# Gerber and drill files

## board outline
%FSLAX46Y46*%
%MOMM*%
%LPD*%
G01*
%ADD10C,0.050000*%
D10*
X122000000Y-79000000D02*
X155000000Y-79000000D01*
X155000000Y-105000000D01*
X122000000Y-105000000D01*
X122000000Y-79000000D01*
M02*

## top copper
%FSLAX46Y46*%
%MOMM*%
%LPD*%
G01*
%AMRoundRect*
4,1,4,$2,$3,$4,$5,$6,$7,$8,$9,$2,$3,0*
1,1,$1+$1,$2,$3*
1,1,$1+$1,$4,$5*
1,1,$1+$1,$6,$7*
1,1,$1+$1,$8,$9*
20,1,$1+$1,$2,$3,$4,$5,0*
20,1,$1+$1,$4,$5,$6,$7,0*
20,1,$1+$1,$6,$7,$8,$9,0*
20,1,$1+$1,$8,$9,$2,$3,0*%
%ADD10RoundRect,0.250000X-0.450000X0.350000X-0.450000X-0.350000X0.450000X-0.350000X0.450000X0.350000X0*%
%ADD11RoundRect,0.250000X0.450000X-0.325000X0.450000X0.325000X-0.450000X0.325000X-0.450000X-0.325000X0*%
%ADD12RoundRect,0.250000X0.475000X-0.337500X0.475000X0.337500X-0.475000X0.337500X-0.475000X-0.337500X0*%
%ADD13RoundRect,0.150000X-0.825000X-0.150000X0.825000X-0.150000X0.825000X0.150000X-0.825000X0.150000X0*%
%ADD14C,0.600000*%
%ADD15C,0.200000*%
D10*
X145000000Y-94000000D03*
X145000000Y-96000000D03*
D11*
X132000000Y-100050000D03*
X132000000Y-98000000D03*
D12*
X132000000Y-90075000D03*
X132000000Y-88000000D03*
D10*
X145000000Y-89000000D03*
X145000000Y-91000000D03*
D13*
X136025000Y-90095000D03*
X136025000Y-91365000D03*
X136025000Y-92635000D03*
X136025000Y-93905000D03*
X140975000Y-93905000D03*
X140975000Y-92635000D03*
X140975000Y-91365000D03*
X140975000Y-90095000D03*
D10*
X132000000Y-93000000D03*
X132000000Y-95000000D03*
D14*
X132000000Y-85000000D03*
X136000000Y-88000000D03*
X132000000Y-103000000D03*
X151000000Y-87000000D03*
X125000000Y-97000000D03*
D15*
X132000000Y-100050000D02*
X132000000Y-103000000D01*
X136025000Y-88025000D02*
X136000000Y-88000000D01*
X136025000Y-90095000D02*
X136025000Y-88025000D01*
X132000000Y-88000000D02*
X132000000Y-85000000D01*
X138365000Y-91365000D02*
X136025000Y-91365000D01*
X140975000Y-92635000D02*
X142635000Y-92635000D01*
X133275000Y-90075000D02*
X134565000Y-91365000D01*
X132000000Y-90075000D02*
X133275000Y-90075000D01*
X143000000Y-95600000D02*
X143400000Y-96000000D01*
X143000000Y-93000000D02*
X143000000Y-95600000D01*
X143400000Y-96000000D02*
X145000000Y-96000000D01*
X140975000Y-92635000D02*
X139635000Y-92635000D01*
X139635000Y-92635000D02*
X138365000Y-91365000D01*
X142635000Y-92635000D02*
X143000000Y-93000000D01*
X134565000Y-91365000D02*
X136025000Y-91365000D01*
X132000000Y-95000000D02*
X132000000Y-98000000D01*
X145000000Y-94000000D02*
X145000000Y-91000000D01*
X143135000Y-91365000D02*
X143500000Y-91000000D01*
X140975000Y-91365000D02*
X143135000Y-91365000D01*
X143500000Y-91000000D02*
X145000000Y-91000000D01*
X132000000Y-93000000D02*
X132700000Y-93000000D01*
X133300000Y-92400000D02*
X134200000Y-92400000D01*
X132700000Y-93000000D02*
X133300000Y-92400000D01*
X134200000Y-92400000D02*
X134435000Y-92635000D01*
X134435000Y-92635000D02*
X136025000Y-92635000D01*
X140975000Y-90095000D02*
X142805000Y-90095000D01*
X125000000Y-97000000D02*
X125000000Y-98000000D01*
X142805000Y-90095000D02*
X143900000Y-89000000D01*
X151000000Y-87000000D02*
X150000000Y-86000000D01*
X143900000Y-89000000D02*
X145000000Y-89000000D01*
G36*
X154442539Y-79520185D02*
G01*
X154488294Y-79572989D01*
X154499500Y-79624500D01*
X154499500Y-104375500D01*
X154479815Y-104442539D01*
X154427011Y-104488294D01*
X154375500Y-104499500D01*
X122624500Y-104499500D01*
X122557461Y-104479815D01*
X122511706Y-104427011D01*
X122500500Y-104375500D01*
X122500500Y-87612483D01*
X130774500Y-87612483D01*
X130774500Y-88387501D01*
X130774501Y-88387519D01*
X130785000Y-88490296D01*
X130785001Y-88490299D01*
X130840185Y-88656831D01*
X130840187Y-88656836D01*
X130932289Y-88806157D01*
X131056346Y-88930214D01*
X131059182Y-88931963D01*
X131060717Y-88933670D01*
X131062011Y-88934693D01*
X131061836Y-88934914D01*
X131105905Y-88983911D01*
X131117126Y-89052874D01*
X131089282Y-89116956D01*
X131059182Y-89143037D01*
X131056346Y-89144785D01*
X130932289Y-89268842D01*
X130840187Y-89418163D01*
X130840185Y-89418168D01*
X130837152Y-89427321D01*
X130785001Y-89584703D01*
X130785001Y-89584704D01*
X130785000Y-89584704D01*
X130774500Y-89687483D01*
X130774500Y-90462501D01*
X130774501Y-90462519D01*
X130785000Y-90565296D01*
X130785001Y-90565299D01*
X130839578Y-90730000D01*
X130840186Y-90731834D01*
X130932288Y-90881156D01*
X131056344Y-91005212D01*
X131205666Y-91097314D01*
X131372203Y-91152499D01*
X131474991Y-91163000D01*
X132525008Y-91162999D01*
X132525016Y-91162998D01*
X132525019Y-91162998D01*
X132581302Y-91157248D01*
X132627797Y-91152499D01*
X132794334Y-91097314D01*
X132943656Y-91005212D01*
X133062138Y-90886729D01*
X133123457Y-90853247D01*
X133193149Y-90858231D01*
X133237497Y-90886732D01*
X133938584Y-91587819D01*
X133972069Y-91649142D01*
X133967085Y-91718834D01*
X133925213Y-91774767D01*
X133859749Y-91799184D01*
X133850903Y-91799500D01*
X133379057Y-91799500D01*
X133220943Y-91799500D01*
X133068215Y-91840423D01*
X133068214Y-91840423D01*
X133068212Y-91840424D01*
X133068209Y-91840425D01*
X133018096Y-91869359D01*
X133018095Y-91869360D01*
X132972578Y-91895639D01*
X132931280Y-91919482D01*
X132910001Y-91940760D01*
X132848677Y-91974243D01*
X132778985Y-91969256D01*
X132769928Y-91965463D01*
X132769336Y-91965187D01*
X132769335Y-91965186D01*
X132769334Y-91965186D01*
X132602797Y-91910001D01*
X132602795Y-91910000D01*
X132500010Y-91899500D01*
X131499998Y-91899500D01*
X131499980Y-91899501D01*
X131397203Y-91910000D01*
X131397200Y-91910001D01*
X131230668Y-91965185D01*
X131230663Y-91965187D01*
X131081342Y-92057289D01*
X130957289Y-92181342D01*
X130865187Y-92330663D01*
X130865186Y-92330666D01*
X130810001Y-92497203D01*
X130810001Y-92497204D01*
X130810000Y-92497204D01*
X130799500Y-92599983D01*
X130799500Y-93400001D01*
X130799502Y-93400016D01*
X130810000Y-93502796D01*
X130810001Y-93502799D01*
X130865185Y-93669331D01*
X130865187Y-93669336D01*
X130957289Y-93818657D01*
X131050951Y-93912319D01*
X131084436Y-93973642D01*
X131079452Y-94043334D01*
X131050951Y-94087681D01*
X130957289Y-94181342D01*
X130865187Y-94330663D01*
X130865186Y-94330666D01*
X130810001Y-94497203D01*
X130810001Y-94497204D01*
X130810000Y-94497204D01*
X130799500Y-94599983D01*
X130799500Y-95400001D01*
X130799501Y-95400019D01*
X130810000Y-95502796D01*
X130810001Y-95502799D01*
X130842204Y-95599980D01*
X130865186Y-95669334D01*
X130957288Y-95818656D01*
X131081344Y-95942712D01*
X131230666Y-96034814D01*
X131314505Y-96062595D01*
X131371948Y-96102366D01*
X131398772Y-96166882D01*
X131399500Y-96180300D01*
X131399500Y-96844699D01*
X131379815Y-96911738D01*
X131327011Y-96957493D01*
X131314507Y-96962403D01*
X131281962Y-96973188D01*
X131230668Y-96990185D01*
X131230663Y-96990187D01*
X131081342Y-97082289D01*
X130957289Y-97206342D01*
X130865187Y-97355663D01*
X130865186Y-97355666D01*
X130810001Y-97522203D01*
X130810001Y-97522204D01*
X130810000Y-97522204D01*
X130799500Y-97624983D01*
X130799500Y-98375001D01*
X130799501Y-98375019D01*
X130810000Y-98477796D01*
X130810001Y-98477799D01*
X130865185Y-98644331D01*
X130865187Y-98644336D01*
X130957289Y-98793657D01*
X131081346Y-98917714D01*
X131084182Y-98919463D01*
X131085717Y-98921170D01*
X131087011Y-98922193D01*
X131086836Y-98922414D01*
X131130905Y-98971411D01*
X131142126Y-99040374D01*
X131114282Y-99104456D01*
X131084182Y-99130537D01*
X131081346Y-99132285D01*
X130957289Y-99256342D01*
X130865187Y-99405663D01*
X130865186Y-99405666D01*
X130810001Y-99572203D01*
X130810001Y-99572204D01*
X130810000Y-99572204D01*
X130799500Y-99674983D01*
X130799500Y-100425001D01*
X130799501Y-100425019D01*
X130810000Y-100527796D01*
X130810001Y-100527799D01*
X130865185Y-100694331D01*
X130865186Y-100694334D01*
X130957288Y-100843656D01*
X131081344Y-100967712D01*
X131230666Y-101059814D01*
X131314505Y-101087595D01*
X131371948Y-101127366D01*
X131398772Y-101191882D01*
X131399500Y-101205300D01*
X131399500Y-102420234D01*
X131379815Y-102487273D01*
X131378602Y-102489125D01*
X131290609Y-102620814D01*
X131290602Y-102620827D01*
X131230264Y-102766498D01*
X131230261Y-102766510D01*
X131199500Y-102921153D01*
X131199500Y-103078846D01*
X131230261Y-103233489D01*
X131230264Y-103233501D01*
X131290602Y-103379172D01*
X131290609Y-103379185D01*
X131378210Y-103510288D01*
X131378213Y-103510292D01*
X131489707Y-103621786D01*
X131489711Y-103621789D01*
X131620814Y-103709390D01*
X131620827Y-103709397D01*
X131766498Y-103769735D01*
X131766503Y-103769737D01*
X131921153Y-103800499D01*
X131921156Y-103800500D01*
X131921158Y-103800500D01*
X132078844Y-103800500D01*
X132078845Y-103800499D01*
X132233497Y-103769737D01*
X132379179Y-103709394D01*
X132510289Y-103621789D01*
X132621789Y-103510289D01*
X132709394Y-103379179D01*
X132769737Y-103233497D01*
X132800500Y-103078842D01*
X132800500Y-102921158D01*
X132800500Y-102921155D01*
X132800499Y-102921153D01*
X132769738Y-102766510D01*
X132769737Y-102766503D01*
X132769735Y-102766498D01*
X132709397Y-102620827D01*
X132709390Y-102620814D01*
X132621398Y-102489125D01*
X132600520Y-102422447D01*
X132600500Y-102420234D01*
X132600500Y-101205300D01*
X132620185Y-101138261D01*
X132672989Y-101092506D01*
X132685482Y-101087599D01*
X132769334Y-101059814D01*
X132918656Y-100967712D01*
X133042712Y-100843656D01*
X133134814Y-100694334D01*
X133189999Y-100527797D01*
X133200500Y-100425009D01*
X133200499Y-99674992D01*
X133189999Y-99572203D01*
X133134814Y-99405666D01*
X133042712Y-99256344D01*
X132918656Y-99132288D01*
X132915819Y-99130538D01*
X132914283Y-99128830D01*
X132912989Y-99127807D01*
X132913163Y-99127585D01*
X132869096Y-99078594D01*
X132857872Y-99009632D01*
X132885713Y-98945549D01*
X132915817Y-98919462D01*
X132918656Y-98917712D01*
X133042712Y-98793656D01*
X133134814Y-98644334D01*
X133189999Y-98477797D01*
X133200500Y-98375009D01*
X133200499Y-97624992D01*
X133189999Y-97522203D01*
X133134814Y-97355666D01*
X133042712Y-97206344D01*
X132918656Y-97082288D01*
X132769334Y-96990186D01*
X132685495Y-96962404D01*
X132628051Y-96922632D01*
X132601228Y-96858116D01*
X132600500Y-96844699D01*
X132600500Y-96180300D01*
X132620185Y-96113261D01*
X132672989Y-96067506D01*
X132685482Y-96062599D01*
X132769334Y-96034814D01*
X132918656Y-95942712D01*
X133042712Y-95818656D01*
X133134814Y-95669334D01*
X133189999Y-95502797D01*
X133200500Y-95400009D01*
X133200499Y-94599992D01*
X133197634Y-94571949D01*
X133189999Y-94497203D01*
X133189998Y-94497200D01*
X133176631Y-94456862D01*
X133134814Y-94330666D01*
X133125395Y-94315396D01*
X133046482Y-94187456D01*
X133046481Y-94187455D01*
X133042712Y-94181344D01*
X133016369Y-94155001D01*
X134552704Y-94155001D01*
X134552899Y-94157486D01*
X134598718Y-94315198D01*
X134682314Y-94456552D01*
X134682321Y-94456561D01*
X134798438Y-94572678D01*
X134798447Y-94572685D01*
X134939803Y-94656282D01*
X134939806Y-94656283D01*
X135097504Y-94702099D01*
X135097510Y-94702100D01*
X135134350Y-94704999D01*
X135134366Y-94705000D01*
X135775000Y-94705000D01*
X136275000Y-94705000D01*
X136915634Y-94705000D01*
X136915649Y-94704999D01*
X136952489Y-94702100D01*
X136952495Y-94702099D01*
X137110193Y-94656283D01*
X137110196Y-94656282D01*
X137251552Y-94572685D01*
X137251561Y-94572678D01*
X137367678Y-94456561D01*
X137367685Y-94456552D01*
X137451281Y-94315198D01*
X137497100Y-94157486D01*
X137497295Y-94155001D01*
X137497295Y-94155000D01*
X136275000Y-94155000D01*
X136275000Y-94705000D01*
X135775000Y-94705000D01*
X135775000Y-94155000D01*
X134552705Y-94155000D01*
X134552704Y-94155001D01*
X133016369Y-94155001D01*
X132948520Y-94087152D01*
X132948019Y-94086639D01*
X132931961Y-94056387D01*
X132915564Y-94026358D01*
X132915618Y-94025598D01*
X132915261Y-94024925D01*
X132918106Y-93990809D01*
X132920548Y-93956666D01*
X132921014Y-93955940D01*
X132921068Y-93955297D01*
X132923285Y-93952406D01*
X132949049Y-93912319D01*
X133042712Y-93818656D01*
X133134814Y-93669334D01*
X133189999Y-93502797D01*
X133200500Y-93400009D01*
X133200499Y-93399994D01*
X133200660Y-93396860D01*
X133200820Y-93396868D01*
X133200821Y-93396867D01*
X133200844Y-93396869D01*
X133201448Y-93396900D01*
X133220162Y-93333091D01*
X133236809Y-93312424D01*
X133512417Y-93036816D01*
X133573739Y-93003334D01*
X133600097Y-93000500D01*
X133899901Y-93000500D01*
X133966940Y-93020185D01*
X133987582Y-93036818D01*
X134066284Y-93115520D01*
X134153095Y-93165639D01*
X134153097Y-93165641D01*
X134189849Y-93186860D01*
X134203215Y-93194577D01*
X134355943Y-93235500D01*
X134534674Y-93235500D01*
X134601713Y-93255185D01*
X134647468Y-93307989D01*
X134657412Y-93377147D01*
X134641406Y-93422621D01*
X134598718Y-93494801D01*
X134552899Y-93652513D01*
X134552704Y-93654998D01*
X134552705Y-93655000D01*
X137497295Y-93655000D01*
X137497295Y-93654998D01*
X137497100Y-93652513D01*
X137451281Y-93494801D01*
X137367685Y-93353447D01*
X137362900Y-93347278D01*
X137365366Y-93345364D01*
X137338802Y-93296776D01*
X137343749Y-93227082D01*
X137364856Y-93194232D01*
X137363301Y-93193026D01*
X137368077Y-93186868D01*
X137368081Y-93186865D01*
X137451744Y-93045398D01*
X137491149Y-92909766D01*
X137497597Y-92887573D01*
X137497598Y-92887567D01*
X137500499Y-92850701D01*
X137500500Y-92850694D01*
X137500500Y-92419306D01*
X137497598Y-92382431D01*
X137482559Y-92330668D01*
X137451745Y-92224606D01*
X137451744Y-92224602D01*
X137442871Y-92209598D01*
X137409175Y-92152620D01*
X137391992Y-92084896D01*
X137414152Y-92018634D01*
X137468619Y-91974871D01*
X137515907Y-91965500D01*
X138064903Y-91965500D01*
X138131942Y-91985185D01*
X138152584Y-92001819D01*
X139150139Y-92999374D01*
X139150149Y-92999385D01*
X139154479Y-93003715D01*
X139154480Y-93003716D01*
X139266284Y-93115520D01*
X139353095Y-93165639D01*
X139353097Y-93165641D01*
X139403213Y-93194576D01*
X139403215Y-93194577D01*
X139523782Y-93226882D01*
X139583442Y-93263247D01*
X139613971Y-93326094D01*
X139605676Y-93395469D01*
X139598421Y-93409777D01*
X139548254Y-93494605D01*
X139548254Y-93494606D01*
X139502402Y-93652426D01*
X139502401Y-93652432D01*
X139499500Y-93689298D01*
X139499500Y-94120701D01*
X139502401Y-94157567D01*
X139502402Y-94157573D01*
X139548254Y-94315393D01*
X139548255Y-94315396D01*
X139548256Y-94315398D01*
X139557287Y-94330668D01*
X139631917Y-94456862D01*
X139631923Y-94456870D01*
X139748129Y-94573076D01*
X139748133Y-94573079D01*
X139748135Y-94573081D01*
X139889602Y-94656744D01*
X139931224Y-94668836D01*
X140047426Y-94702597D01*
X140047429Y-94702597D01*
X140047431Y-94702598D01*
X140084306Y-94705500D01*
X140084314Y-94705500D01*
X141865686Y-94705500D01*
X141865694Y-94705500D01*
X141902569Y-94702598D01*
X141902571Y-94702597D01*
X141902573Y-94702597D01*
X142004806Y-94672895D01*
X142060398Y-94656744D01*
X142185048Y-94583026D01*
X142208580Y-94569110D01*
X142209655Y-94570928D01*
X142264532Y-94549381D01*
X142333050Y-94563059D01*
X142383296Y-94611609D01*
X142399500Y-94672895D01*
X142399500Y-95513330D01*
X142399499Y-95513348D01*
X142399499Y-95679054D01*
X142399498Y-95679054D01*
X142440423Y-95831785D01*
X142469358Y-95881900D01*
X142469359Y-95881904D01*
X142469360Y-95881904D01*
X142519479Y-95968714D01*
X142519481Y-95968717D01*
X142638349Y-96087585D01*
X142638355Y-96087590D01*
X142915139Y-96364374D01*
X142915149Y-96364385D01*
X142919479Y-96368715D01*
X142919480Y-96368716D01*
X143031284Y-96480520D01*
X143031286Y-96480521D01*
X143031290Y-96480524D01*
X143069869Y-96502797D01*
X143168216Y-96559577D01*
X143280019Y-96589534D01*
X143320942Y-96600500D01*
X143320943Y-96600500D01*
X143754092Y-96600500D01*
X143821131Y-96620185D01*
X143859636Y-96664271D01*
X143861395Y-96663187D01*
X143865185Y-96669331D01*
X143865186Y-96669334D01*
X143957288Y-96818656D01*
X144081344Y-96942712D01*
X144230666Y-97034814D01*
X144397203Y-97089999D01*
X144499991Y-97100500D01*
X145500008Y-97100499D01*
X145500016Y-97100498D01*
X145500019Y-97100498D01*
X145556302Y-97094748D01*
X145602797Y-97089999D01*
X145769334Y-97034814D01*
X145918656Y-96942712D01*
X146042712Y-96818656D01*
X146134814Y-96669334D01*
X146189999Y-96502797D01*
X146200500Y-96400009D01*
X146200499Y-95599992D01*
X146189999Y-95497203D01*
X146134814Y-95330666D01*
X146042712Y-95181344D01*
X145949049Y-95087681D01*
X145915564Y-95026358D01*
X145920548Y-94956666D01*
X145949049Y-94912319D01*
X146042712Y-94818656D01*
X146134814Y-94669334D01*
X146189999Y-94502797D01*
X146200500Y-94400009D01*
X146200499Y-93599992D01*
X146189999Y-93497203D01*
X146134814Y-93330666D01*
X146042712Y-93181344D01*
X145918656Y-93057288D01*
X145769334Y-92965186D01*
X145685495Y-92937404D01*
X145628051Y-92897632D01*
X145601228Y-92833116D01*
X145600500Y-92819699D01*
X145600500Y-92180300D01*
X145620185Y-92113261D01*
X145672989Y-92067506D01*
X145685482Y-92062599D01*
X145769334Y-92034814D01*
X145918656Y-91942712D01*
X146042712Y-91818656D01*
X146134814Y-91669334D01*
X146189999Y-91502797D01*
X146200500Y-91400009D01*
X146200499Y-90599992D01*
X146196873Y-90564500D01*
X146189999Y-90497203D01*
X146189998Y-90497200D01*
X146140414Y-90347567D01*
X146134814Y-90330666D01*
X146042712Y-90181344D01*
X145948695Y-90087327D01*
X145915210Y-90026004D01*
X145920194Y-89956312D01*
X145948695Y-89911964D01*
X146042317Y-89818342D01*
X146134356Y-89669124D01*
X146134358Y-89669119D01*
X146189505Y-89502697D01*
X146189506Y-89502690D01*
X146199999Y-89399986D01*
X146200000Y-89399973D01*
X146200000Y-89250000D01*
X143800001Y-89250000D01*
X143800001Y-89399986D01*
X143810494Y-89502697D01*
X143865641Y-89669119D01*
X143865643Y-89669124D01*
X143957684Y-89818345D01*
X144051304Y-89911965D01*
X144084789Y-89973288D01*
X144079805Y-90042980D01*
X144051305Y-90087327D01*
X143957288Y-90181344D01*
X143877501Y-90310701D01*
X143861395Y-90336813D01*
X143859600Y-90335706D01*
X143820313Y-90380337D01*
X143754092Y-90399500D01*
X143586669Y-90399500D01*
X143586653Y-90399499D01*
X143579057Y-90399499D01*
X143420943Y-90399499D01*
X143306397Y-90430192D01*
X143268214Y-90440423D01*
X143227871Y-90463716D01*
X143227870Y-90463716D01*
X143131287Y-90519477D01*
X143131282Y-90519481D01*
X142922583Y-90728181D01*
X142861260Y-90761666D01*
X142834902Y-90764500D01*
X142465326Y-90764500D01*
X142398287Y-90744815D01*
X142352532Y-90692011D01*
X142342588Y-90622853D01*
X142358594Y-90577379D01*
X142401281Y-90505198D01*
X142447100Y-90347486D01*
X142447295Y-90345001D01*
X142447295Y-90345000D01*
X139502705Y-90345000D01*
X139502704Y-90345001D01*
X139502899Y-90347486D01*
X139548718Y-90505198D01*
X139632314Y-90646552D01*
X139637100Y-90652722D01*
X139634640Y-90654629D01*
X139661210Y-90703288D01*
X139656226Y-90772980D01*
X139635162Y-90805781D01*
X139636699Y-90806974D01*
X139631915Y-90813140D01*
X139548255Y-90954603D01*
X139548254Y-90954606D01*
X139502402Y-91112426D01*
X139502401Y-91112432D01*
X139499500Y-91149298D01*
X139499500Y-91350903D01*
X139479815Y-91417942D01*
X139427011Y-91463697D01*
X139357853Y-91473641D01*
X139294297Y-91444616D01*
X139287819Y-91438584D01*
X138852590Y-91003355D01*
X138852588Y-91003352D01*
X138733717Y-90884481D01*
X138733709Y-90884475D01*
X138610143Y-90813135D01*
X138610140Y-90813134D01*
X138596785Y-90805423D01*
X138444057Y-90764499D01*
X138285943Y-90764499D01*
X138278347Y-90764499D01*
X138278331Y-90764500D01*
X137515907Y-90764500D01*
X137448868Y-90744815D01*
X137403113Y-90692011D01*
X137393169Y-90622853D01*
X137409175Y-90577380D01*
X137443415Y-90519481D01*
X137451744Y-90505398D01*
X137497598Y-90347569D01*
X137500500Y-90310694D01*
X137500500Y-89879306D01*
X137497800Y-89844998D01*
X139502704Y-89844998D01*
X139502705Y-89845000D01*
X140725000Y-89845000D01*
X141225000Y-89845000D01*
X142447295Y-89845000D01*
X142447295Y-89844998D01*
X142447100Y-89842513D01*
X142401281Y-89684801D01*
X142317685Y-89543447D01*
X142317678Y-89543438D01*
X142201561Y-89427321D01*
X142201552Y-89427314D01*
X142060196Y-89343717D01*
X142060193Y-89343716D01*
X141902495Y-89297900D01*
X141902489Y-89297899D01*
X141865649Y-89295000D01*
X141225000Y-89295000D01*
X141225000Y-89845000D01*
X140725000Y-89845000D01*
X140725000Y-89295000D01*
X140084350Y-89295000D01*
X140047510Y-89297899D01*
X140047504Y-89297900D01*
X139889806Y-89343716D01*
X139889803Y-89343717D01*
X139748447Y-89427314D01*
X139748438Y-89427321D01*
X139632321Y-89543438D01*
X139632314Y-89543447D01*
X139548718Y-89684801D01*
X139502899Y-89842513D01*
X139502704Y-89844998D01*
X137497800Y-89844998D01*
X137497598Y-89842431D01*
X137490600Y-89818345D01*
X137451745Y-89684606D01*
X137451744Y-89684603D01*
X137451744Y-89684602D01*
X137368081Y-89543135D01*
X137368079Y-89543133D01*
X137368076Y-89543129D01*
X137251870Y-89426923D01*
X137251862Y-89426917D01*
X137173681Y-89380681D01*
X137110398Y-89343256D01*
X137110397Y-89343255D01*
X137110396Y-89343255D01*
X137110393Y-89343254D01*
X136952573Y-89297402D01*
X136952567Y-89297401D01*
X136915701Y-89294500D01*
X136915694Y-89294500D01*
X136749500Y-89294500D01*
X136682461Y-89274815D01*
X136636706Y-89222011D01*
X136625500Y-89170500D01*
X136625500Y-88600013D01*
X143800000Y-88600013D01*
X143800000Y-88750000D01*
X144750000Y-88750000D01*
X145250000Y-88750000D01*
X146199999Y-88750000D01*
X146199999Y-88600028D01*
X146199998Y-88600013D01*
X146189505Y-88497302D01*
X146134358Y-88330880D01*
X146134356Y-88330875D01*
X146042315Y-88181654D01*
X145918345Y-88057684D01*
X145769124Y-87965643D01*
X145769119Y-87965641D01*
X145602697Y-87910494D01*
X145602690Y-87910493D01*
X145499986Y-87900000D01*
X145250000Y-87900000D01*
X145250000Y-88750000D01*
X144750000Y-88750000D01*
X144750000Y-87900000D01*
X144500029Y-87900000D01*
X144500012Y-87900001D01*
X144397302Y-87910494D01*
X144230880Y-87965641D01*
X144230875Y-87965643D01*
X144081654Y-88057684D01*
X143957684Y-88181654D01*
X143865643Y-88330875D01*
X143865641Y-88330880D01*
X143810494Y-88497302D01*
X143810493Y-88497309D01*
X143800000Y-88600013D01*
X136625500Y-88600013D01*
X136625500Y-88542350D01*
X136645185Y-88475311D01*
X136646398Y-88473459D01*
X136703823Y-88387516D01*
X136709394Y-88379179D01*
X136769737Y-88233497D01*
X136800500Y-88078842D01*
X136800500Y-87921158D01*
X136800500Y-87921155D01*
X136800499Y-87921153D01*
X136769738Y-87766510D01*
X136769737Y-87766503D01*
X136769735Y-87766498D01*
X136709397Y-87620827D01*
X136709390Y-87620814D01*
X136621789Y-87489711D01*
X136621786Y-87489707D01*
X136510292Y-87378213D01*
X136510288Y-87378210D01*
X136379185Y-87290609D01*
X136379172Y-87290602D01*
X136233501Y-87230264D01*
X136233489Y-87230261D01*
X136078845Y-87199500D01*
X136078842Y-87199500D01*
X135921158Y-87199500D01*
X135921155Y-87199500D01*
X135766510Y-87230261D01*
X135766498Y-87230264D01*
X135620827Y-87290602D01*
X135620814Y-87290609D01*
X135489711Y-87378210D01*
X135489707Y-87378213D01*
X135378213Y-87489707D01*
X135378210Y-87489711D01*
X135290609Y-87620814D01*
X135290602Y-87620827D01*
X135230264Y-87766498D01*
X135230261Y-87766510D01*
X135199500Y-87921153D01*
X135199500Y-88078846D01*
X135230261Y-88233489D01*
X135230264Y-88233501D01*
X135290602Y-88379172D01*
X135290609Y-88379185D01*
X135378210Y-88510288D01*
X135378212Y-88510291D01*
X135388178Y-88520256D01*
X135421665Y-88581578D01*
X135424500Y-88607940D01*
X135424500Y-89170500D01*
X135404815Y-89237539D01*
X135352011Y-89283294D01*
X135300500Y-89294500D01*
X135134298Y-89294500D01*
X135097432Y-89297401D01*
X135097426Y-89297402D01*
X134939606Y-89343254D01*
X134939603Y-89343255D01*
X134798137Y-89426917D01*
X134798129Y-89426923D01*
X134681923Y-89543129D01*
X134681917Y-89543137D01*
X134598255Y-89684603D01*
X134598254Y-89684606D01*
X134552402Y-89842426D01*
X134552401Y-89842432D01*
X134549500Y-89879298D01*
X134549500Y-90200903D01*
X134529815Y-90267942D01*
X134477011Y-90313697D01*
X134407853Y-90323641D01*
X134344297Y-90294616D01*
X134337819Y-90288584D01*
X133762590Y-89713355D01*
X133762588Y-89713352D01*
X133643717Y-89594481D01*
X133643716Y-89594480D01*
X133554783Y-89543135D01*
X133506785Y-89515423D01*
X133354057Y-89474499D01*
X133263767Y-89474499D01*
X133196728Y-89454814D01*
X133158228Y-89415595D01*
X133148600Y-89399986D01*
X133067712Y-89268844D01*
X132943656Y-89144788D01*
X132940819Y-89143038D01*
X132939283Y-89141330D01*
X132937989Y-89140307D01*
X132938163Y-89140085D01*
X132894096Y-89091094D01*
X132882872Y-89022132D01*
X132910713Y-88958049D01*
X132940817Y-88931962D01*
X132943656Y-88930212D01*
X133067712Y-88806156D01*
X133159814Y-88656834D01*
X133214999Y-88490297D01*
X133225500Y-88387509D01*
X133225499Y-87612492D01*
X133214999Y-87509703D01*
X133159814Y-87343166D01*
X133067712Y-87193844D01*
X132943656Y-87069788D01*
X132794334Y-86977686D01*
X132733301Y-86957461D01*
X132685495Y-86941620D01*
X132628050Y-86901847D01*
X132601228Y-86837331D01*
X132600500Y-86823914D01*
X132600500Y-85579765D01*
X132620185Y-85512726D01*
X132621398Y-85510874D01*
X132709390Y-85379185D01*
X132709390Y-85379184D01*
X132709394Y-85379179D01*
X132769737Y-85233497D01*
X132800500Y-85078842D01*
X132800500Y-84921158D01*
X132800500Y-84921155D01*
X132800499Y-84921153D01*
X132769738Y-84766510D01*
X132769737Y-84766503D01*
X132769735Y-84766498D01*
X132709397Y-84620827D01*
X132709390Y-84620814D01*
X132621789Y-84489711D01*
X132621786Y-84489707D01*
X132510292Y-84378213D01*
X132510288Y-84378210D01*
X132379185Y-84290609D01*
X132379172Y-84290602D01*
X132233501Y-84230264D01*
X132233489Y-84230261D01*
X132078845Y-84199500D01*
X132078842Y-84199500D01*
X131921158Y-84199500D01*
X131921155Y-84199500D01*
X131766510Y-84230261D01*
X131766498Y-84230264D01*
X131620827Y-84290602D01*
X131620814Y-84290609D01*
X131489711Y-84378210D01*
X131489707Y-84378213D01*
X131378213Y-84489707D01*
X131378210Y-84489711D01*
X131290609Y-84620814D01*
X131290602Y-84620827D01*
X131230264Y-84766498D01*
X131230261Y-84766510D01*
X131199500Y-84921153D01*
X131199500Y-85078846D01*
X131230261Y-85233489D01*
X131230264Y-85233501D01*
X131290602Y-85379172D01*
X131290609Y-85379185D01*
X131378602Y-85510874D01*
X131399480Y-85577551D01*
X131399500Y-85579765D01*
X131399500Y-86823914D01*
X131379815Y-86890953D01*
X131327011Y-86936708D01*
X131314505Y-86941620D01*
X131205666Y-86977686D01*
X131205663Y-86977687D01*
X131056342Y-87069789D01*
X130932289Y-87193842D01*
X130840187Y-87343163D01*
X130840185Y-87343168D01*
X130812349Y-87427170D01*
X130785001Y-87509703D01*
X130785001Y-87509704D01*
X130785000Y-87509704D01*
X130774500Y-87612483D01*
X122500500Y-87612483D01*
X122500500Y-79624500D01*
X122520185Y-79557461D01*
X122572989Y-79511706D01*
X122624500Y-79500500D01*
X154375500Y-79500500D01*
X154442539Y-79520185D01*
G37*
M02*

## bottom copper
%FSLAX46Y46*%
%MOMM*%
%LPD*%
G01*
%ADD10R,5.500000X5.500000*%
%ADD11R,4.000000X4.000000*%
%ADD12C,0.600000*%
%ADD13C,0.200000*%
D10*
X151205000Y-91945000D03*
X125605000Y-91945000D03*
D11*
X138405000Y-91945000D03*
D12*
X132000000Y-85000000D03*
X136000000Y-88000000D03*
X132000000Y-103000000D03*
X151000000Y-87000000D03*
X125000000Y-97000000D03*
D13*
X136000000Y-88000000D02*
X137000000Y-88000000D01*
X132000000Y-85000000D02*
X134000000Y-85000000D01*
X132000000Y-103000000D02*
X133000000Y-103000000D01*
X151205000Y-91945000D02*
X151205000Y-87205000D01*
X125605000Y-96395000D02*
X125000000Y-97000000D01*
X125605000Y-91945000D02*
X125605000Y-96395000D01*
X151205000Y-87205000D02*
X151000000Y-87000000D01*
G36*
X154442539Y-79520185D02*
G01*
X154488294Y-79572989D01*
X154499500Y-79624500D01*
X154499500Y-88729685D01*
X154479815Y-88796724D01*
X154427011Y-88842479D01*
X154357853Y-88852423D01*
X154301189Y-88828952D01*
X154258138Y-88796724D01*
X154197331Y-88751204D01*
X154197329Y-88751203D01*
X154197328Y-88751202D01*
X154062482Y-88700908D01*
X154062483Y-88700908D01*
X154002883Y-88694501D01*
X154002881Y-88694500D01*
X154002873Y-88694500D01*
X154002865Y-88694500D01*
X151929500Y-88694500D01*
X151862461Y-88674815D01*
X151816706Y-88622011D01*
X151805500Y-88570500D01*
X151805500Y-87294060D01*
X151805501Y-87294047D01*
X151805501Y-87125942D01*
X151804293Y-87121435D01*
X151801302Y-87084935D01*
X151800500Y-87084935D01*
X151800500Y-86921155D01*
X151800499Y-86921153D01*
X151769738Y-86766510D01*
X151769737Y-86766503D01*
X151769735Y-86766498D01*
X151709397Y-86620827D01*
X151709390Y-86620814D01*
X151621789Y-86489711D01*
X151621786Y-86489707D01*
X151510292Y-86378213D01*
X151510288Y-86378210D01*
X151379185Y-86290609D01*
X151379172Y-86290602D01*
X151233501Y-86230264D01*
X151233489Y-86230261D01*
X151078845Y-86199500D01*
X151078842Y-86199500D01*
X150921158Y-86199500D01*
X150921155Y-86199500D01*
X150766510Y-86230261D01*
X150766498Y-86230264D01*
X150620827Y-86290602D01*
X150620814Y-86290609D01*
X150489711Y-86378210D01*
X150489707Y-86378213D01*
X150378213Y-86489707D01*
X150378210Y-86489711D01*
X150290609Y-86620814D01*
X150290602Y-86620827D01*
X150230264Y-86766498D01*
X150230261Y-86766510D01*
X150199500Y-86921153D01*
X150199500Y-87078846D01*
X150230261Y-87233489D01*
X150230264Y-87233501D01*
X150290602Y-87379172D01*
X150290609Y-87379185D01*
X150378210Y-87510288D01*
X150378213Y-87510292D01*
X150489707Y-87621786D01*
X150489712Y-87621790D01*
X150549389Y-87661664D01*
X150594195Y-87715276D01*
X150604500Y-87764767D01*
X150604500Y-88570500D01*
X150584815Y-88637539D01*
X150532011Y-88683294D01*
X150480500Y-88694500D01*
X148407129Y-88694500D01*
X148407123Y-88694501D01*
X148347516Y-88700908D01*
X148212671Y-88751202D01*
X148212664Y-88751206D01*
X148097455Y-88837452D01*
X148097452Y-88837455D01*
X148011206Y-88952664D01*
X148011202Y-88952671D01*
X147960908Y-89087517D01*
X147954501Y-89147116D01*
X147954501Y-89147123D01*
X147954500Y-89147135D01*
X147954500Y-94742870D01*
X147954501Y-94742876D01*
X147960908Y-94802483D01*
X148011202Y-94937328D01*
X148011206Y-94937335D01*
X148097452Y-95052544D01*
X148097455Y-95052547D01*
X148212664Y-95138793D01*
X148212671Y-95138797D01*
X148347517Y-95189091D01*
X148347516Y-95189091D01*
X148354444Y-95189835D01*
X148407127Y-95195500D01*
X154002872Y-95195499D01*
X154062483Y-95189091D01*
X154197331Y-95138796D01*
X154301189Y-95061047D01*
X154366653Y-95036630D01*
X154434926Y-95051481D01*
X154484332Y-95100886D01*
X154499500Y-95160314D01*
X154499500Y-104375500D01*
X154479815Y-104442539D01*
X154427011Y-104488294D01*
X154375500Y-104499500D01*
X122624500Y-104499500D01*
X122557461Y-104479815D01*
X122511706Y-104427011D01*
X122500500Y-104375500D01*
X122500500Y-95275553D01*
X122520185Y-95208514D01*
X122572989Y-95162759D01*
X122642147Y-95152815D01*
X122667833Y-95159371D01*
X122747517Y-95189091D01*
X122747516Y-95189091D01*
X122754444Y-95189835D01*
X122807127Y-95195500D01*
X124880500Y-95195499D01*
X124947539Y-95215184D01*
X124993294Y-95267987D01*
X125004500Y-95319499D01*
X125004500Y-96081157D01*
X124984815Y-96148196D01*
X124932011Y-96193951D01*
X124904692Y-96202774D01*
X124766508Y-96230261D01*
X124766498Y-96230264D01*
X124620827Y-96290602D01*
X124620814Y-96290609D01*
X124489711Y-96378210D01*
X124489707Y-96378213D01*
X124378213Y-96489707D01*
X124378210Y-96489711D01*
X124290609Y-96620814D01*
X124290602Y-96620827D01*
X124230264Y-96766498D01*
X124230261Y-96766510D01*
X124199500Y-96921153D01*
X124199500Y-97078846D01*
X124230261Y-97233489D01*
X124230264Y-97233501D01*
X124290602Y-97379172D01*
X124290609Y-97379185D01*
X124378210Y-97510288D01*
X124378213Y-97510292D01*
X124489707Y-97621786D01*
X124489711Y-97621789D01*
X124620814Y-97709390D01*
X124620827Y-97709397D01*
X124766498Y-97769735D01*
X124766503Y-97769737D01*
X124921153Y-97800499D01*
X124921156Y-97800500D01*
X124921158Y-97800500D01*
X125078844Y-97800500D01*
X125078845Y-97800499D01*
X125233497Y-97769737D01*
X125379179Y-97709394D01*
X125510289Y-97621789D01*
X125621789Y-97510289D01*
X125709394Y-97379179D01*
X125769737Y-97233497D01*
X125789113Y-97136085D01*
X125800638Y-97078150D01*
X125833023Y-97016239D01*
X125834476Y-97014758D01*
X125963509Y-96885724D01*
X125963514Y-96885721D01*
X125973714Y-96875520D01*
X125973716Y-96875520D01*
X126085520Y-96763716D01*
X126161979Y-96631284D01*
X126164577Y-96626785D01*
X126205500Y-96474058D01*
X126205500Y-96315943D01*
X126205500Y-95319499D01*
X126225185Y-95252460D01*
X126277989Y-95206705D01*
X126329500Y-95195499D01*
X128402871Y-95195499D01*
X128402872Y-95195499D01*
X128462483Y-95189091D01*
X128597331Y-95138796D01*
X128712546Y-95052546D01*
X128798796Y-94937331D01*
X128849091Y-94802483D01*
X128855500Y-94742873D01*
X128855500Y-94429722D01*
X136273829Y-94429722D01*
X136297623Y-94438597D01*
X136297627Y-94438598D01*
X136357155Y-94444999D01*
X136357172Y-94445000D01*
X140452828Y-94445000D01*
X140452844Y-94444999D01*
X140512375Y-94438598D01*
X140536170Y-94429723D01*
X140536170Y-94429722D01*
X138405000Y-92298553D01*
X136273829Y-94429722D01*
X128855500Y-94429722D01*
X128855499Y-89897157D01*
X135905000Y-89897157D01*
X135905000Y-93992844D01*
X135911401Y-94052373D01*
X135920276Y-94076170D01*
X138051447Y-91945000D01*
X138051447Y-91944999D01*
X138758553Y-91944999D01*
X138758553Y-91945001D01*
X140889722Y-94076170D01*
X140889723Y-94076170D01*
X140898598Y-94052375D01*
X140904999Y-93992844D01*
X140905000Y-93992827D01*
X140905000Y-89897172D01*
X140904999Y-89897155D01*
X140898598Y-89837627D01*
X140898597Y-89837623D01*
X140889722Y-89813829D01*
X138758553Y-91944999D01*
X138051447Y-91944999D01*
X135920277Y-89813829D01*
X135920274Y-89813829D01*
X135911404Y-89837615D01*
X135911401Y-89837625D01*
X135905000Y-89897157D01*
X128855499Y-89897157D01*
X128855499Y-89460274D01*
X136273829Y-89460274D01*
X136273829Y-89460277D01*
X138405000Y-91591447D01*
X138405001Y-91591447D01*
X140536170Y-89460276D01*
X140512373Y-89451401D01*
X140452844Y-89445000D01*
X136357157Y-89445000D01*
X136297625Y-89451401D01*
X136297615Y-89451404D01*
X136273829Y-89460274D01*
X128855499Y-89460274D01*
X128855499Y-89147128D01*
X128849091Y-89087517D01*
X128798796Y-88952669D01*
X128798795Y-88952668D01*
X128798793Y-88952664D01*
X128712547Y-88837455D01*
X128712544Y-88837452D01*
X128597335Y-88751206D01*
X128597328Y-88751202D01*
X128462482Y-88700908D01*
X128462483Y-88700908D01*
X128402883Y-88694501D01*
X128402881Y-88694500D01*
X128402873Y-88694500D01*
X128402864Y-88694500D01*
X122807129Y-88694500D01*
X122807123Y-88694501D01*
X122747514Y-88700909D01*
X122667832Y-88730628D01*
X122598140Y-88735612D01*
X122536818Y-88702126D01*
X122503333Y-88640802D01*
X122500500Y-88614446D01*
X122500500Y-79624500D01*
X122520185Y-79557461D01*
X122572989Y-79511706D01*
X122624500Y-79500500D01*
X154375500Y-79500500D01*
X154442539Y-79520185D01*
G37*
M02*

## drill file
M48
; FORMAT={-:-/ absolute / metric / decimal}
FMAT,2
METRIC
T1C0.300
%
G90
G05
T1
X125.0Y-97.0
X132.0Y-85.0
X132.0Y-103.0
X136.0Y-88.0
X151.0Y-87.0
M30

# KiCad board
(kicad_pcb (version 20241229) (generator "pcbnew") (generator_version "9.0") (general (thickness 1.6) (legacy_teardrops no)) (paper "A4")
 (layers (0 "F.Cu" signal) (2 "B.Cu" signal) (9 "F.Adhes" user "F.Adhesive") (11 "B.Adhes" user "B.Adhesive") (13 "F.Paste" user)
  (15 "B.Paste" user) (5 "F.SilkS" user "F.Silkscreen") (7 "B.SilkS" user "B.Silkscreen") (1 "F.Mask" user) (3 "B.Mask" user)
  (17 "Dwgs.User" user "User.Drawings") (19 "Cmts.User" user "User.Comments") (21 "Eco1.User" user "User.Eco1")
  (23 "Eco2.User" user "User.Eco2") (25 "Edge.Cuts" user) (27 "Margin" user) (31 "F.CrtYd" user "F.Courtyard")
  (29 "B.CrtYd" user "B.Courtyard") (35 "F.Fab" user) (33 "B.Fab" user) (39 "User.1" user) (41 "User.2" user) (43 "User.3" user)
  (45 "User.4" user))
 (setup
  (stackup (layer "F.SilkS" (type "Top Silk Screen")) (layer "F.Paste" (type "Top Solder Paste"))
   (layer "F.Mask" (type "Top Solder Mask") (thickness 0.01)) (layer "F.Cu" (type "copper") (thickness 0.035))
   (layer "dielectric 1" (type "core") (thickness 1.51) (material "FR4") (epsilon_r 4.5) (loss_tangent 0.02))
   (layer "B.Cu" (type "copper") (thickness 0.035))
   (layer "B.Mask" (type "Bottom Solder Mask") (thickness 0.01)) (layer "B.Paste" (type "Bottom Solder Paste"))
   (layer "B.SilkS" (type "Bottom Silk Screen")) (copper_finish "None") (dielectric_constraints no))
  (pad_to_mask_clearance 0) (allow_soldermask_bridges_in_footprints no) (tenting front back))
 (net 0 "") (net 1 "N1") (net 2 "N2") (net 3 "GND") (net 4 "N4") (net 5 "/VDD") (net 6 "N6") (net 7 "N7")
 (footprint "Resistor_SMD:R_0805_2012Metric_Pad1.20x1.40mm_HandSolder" (layer "F.Cu") (at 145 95 -90)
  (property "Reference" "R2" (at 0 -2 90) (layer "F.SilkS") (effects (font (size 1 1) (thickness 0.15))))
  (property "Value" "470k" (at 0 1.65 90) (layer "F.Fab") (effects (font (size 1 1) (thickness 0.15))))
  (pad "1" smd roundrect (at -1 0 270) (size 1.2 1.4) (layers "F.Cu" "F.Mask" "F.Paste") (roundrect_rratio 0.208333) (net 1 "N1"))
  (pad "2" smd roundrect (at 1 0 270) (size 1.2 1.4) (layers "F.Cu" "F.Mask" "F.Paste") (roundrect_rratio 0.208333) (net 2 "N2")))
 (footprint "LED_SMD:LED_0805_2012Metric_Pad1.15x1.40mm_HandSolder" (layer "F.Cu") (at 132 99.025 90)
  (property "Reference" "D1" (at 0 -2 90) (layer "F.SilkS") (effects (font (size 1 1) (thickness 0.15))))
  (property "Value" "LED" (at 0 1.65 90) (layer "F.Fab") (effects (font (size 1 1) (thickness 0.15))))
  (pad "1" smd roundrect (at -1.025 0 90) (size 1.15 1.4) (layers "F.Cu" "F.Mask" "F.Paste") (roundrect_rratio 0.217391) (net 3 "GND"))
  (pad "2" smd roundrect (at 1.025 0 90) (size 1.15 1.4) (layers "F.Cu" "F.Mask" "F.Paste") (roundrect_rratio 0.217391) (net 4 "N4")))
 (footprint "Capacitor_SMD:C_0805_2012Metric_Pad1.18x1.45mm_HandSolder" (layer "F.Cu") (at 132 89.0375 90)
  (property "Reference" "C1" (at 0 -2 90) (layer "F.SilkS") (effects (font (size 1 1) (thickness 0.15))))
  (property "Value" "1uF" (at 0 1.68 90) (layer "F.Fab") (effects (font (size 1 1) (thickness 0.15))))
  (pad "1" smd roundrect (at -1.0375 0 90) (size 1.175 1.45) (layers "F.Cu" "F.Mask" "F.Paste") (roundrect_rratio 0.212766) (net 2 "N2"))
  (pad "2" smd roundrect (at 1.0375 0 90) (size 1.175 1.45) (layers "F.Cu" "F.Mask" "F.Paste") (roundrect_rratio 0.212766) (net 3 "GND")))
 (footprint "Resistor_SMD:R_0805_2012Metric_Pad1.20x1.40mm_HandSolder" (layer "F.Cu") (at 145 90 -90)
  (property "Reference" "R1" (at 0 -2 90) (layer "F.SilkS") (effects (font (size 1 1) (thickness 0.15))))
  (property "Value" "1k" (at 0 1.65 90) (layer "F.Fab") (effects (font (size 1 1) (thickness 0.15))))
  (pad "1" smd roundrect (at -1 0 270) (size 1.2 1.4) (layers "F.Cu" "F.Mask" "F.Paste") (roundrect_rratio 0.208333) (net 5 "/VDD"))
  (pad "2" smd roundrect (at 1 0 270) (size 1.2 1.4) (layers "F.Cu" "F.Mask" "F.Paste") (roundrect_rratio 0.208333) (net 1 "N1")))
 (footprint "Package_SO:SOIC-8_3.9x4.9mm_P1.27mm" (layer "F.Cu") (at 138.5 92)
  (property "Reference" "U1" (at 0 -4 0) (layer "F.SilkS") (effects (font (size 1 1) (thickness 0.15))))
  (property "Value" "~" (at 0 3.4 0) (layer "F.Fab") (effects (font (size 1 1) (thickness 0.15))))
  (pad "1" smd roundrect (at -2.475 -1.905) (size 1.95 0.6) (layers "F.Cu" "F.Mask" "F.Paste") (roundrect_rratio 0.25) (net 3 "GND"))
  (pad "2" smd roundrect (at -2.475 -0.635) (size 1.95 0.6) (layers "F.Cu" "F.Mask" "F.Paste") (roundrect_rratio 0.25) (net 2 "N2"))
  (pad "3" smd roundrect (at -2.475 0.635) (size 1.95 0.6) (layers "F.Cu" "F.Mask" "F.Paste") (roundrect_rratio 0.25) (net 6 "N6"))
  (pad "4" smd roundrect (at -2.475 1.905) (size 1.95 0.6) (layers "F.Cu" "F.Mask" "F.Paste") (roundrect_rratio 0.25) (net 5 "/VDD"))
  (pad "5" smd roundrect (at 2.475 1.905) (size 1.95 0.6) (layers "F.Cu" "F.Mask" "F.Paste") (roundrect_rratio 0.25) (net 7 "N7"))
  (pad "6" smd roundrect (at 2.475 0.635) (size 1.95 0.6) (layers "F.Cu" "F.Mask" "F.Paste") (roundrect_rratio 0.25) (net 2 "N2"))
  (pad "7" smd roundrect (at 2.475 -0.635) (size 1.95 0.6) (layers "F.Cu" "F.Mask" "F.Paste") (roundrect_rratio 0.25) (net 1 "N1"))
  (pad "8" smd roundrect (at 2.475 -1.905) (size 1.95 0.6) (layers "F.Cu" "F.Mask" "F.Paste") (roundrect_rratio 0.25) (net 5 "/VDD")))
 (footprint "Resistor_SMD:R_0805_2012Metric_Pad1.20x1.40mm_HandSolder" (layer "F.Cu") (at 132 94 -90)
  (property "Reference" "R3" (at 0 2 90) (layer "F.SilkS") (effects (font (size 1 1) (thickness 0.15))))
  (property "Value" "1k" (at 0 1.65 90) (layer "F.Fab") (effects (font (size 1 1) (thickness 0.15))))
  (pad "1" smd roundrect (at -1 0 270) (size 1.2 1.4) (layers "F.Cu" "F.Mask" "F.Paste") (roundrect_rratio 0.208333) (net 6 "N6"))
  (pad "2" smd roundrect (at 1 0 270) (size 1.2 1.4) (layers "F.Cu" "F.Mask" "F.Paste") (roundrect_rratio 0.208333) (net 4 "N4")))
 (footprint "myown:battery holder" (layer "B.Cu") (at 138.405 91.945 180)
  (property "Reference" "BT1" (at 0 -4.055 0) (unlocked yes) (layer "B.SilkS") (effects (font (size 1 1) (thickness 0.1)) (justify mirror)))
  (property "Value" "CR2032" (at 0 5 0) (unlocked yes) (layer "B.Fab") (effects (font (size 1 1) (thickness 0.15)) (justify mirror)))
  (pad "1" smd rect (at -12.8 0 180) (size 5.5 5.5) (layers "B.Cu" "B.Mask" "B.Paste") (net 5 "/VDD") (thermal_bridge_angle 45))
  (pad "1" smd rect (at 12.8 0 180) (size 5.5 5.5) (layers "B.Cu" "B.Mask" "B.Paste") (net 5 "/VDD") (thermal_bridge_angle 45))
  (pad "2" smd rect (at 0 0 180) (size 4 4) (layers "B.Cu" "B.Mask" "B.Paste") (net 3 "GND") (thermal_bridge_angle 45)))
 (gr_rect (start 122 79) (end 155 105) (stroke (width 0.05) (type default)) (fill no) (layer "Edge.Cuts"))
 (segment (start 132 100.05) (end 132 103) (width 0.2) (layer "F.Cu") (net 3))
 (segment (start 136.025 88.025) (end 136 88) (width 0.2) (layer "F.Cu") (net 3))
 (segment (start 136.025 90.095) (end 136.025 88.025) (width 0.2) (layer "F.Cu") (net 3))
 (segment (start 132 88) (end 132 85) (width 0.2) (layer "F.Cu") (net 3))
 (via (at 132 85) (size 0.6) (drill 0.3) (layers "F.Cu" "B.Cu") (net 3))
 (via (at 136 88) (size 0.6) (drill 0.3) (layers "F.Cu" "B.Cu") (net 3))
 (via (at 132 103) (size 0.6) (drill 0.3) (layers "F.Cu" "B.Cu") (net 3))
 (segment (start 136 88) (end 137 88) (width 0.2) (layer "B.Cu") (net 3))
 (segment (start 132 85) (end 134 85) (width 0.2) (layer "B.Cu") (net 3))
 (segment (start 132 103) (end 133 103) (width 0.2) (layer "B.Cu") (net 3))
 (segment (start 138.365 91.365) (end 136.025 91.365) (width 0.2) (layer "F.Cu") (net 2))
 (segment (start 140.975 92.635) (end 142.635 92.635) (width 0.2) (layer "F.Cu") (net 2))
 (segment (start 133.275 90.075) (end 134.565 91.365) (width 0.2) (layer "F.Cu") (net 2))
 (segment (start 132 90.075) (end 133.275 90.075) (width 0.2) (layer "F.Cu") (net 2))
 (segment (start 143 95.6) (end 143.4 96) (width 0.2) (layer "F.Cu") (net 2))
 (segment (start 143 93) (end 143 95.6) (width 0.2) (layer "F.Cu") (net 2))
 (segment (start 143.4 96) (end 145 96) (width 0.2) (layer "F.Cu") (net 2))
 (segment (start 140.975 92.635) (end 139.635 92.635) (width 0.2) (layer "F.Cu") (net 2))
 (segment (start 139.635 92.635) (end 138.365 91.365) (width 0.2) (layer "F.Cu") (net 2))
 (segment (start 142.635 92.635) (end 143 93) (width 0.2) (layer "F.Cu") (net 2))
 (segment (start 134.565 91.365) (end 136.025 91.365) (width 0.2) (layer "F.Cu") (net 2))
 (segment (start 132 95) (end 132 98) (width 0.2) (layer "F.Cu") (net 4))
 (segment (start 145 94) (end 145 91) (width 0.2) (layer "F.Cu") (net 1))
 (segment (start 143.135 91.365) (end 143.5 91) (width 0.2) (layer "F.Cu") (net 1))
 (segment (start 140.975 91.365) (end 143.135 91.365) (width 0.2) (layer "F.Cu") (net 1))
 (segment (start 143.5 91) (end 145 91) (width 0.2) (layer "F.Cu") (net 1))
 (segment (start 132 93) (end 132.7 93) (width 0.2) (layer "F.Cu") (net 6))
 (segment (start 133.3 92.4) (end 134.2 92.4) (width 0.2) (layer "F.Cu") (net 6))
 (segment (start 132.7 93) (end 133.3 92.4) (width 0.2) (layer "F.Cu") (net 6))
 (segment (start 134.2 92.4) (end 134.435 92.635) (width 0.2) (layer "F.Cu") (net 6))
 (segment (start 134.435 92.635) (end 136.025 92.635) (width 0.2) (layer "F.Cu") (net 6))
 (segment (start 140.975 90.095) (end 142.805 90.095) (width 0.2) (layer "F.Cu") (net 5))
 (segment (start 125 97) (end 125 98) (width 0.2) (layer "F.Cu") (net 5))
 (segment (start 142.805 90.095) (end 143.9 89) (width 0.2) (layer "F.Cu") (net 5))
 (segment (start 151 87) (end 150 86) (width 0.2) (layer "F.Cu") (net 5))
 (segment (start 143.9 89) (end 145 89) (width 0.2) (layer "F.Cu") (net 5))
 (via (at 151 87) (size 0.6) (drill 0.3) (layers "F.Cu" "B.Cu") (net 5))
 (via (at 125 97) (size 0.6) (drill 0.3) (layers "F.Cu" "B.Cu") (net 5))
 (segment (start 151.205 91.945) (end 151.205 87.205) (width 0.2) (layer "B.Cu") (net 5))
 (segment (start 125.605 96.395) (end 125 97) (width 0.2) (layer "B.Cu") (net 5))
 (segment (start 125.605 91.945) (end 125.605 96.395) (width 0.2) (layer "B.Cu") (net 5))
 (segment (start 151.205 87.205) (end 151 87) (width 0.2) (layer "B.Cu") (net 5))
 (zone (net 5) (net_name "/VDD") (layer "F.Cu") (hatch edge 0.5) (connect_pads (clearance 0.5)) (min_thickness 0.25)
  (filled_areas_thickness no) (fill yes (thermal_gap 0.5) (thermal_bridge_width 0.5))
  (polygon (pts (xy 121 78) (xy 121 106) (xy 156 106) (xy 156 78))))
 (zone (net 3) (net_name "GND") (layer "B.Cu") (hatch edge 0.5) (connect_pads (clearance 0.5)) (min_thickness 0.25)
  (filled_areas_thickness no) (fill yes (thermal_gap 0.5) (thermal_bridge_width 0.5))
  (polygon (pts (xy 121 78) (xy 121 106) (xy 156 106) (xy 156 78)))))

